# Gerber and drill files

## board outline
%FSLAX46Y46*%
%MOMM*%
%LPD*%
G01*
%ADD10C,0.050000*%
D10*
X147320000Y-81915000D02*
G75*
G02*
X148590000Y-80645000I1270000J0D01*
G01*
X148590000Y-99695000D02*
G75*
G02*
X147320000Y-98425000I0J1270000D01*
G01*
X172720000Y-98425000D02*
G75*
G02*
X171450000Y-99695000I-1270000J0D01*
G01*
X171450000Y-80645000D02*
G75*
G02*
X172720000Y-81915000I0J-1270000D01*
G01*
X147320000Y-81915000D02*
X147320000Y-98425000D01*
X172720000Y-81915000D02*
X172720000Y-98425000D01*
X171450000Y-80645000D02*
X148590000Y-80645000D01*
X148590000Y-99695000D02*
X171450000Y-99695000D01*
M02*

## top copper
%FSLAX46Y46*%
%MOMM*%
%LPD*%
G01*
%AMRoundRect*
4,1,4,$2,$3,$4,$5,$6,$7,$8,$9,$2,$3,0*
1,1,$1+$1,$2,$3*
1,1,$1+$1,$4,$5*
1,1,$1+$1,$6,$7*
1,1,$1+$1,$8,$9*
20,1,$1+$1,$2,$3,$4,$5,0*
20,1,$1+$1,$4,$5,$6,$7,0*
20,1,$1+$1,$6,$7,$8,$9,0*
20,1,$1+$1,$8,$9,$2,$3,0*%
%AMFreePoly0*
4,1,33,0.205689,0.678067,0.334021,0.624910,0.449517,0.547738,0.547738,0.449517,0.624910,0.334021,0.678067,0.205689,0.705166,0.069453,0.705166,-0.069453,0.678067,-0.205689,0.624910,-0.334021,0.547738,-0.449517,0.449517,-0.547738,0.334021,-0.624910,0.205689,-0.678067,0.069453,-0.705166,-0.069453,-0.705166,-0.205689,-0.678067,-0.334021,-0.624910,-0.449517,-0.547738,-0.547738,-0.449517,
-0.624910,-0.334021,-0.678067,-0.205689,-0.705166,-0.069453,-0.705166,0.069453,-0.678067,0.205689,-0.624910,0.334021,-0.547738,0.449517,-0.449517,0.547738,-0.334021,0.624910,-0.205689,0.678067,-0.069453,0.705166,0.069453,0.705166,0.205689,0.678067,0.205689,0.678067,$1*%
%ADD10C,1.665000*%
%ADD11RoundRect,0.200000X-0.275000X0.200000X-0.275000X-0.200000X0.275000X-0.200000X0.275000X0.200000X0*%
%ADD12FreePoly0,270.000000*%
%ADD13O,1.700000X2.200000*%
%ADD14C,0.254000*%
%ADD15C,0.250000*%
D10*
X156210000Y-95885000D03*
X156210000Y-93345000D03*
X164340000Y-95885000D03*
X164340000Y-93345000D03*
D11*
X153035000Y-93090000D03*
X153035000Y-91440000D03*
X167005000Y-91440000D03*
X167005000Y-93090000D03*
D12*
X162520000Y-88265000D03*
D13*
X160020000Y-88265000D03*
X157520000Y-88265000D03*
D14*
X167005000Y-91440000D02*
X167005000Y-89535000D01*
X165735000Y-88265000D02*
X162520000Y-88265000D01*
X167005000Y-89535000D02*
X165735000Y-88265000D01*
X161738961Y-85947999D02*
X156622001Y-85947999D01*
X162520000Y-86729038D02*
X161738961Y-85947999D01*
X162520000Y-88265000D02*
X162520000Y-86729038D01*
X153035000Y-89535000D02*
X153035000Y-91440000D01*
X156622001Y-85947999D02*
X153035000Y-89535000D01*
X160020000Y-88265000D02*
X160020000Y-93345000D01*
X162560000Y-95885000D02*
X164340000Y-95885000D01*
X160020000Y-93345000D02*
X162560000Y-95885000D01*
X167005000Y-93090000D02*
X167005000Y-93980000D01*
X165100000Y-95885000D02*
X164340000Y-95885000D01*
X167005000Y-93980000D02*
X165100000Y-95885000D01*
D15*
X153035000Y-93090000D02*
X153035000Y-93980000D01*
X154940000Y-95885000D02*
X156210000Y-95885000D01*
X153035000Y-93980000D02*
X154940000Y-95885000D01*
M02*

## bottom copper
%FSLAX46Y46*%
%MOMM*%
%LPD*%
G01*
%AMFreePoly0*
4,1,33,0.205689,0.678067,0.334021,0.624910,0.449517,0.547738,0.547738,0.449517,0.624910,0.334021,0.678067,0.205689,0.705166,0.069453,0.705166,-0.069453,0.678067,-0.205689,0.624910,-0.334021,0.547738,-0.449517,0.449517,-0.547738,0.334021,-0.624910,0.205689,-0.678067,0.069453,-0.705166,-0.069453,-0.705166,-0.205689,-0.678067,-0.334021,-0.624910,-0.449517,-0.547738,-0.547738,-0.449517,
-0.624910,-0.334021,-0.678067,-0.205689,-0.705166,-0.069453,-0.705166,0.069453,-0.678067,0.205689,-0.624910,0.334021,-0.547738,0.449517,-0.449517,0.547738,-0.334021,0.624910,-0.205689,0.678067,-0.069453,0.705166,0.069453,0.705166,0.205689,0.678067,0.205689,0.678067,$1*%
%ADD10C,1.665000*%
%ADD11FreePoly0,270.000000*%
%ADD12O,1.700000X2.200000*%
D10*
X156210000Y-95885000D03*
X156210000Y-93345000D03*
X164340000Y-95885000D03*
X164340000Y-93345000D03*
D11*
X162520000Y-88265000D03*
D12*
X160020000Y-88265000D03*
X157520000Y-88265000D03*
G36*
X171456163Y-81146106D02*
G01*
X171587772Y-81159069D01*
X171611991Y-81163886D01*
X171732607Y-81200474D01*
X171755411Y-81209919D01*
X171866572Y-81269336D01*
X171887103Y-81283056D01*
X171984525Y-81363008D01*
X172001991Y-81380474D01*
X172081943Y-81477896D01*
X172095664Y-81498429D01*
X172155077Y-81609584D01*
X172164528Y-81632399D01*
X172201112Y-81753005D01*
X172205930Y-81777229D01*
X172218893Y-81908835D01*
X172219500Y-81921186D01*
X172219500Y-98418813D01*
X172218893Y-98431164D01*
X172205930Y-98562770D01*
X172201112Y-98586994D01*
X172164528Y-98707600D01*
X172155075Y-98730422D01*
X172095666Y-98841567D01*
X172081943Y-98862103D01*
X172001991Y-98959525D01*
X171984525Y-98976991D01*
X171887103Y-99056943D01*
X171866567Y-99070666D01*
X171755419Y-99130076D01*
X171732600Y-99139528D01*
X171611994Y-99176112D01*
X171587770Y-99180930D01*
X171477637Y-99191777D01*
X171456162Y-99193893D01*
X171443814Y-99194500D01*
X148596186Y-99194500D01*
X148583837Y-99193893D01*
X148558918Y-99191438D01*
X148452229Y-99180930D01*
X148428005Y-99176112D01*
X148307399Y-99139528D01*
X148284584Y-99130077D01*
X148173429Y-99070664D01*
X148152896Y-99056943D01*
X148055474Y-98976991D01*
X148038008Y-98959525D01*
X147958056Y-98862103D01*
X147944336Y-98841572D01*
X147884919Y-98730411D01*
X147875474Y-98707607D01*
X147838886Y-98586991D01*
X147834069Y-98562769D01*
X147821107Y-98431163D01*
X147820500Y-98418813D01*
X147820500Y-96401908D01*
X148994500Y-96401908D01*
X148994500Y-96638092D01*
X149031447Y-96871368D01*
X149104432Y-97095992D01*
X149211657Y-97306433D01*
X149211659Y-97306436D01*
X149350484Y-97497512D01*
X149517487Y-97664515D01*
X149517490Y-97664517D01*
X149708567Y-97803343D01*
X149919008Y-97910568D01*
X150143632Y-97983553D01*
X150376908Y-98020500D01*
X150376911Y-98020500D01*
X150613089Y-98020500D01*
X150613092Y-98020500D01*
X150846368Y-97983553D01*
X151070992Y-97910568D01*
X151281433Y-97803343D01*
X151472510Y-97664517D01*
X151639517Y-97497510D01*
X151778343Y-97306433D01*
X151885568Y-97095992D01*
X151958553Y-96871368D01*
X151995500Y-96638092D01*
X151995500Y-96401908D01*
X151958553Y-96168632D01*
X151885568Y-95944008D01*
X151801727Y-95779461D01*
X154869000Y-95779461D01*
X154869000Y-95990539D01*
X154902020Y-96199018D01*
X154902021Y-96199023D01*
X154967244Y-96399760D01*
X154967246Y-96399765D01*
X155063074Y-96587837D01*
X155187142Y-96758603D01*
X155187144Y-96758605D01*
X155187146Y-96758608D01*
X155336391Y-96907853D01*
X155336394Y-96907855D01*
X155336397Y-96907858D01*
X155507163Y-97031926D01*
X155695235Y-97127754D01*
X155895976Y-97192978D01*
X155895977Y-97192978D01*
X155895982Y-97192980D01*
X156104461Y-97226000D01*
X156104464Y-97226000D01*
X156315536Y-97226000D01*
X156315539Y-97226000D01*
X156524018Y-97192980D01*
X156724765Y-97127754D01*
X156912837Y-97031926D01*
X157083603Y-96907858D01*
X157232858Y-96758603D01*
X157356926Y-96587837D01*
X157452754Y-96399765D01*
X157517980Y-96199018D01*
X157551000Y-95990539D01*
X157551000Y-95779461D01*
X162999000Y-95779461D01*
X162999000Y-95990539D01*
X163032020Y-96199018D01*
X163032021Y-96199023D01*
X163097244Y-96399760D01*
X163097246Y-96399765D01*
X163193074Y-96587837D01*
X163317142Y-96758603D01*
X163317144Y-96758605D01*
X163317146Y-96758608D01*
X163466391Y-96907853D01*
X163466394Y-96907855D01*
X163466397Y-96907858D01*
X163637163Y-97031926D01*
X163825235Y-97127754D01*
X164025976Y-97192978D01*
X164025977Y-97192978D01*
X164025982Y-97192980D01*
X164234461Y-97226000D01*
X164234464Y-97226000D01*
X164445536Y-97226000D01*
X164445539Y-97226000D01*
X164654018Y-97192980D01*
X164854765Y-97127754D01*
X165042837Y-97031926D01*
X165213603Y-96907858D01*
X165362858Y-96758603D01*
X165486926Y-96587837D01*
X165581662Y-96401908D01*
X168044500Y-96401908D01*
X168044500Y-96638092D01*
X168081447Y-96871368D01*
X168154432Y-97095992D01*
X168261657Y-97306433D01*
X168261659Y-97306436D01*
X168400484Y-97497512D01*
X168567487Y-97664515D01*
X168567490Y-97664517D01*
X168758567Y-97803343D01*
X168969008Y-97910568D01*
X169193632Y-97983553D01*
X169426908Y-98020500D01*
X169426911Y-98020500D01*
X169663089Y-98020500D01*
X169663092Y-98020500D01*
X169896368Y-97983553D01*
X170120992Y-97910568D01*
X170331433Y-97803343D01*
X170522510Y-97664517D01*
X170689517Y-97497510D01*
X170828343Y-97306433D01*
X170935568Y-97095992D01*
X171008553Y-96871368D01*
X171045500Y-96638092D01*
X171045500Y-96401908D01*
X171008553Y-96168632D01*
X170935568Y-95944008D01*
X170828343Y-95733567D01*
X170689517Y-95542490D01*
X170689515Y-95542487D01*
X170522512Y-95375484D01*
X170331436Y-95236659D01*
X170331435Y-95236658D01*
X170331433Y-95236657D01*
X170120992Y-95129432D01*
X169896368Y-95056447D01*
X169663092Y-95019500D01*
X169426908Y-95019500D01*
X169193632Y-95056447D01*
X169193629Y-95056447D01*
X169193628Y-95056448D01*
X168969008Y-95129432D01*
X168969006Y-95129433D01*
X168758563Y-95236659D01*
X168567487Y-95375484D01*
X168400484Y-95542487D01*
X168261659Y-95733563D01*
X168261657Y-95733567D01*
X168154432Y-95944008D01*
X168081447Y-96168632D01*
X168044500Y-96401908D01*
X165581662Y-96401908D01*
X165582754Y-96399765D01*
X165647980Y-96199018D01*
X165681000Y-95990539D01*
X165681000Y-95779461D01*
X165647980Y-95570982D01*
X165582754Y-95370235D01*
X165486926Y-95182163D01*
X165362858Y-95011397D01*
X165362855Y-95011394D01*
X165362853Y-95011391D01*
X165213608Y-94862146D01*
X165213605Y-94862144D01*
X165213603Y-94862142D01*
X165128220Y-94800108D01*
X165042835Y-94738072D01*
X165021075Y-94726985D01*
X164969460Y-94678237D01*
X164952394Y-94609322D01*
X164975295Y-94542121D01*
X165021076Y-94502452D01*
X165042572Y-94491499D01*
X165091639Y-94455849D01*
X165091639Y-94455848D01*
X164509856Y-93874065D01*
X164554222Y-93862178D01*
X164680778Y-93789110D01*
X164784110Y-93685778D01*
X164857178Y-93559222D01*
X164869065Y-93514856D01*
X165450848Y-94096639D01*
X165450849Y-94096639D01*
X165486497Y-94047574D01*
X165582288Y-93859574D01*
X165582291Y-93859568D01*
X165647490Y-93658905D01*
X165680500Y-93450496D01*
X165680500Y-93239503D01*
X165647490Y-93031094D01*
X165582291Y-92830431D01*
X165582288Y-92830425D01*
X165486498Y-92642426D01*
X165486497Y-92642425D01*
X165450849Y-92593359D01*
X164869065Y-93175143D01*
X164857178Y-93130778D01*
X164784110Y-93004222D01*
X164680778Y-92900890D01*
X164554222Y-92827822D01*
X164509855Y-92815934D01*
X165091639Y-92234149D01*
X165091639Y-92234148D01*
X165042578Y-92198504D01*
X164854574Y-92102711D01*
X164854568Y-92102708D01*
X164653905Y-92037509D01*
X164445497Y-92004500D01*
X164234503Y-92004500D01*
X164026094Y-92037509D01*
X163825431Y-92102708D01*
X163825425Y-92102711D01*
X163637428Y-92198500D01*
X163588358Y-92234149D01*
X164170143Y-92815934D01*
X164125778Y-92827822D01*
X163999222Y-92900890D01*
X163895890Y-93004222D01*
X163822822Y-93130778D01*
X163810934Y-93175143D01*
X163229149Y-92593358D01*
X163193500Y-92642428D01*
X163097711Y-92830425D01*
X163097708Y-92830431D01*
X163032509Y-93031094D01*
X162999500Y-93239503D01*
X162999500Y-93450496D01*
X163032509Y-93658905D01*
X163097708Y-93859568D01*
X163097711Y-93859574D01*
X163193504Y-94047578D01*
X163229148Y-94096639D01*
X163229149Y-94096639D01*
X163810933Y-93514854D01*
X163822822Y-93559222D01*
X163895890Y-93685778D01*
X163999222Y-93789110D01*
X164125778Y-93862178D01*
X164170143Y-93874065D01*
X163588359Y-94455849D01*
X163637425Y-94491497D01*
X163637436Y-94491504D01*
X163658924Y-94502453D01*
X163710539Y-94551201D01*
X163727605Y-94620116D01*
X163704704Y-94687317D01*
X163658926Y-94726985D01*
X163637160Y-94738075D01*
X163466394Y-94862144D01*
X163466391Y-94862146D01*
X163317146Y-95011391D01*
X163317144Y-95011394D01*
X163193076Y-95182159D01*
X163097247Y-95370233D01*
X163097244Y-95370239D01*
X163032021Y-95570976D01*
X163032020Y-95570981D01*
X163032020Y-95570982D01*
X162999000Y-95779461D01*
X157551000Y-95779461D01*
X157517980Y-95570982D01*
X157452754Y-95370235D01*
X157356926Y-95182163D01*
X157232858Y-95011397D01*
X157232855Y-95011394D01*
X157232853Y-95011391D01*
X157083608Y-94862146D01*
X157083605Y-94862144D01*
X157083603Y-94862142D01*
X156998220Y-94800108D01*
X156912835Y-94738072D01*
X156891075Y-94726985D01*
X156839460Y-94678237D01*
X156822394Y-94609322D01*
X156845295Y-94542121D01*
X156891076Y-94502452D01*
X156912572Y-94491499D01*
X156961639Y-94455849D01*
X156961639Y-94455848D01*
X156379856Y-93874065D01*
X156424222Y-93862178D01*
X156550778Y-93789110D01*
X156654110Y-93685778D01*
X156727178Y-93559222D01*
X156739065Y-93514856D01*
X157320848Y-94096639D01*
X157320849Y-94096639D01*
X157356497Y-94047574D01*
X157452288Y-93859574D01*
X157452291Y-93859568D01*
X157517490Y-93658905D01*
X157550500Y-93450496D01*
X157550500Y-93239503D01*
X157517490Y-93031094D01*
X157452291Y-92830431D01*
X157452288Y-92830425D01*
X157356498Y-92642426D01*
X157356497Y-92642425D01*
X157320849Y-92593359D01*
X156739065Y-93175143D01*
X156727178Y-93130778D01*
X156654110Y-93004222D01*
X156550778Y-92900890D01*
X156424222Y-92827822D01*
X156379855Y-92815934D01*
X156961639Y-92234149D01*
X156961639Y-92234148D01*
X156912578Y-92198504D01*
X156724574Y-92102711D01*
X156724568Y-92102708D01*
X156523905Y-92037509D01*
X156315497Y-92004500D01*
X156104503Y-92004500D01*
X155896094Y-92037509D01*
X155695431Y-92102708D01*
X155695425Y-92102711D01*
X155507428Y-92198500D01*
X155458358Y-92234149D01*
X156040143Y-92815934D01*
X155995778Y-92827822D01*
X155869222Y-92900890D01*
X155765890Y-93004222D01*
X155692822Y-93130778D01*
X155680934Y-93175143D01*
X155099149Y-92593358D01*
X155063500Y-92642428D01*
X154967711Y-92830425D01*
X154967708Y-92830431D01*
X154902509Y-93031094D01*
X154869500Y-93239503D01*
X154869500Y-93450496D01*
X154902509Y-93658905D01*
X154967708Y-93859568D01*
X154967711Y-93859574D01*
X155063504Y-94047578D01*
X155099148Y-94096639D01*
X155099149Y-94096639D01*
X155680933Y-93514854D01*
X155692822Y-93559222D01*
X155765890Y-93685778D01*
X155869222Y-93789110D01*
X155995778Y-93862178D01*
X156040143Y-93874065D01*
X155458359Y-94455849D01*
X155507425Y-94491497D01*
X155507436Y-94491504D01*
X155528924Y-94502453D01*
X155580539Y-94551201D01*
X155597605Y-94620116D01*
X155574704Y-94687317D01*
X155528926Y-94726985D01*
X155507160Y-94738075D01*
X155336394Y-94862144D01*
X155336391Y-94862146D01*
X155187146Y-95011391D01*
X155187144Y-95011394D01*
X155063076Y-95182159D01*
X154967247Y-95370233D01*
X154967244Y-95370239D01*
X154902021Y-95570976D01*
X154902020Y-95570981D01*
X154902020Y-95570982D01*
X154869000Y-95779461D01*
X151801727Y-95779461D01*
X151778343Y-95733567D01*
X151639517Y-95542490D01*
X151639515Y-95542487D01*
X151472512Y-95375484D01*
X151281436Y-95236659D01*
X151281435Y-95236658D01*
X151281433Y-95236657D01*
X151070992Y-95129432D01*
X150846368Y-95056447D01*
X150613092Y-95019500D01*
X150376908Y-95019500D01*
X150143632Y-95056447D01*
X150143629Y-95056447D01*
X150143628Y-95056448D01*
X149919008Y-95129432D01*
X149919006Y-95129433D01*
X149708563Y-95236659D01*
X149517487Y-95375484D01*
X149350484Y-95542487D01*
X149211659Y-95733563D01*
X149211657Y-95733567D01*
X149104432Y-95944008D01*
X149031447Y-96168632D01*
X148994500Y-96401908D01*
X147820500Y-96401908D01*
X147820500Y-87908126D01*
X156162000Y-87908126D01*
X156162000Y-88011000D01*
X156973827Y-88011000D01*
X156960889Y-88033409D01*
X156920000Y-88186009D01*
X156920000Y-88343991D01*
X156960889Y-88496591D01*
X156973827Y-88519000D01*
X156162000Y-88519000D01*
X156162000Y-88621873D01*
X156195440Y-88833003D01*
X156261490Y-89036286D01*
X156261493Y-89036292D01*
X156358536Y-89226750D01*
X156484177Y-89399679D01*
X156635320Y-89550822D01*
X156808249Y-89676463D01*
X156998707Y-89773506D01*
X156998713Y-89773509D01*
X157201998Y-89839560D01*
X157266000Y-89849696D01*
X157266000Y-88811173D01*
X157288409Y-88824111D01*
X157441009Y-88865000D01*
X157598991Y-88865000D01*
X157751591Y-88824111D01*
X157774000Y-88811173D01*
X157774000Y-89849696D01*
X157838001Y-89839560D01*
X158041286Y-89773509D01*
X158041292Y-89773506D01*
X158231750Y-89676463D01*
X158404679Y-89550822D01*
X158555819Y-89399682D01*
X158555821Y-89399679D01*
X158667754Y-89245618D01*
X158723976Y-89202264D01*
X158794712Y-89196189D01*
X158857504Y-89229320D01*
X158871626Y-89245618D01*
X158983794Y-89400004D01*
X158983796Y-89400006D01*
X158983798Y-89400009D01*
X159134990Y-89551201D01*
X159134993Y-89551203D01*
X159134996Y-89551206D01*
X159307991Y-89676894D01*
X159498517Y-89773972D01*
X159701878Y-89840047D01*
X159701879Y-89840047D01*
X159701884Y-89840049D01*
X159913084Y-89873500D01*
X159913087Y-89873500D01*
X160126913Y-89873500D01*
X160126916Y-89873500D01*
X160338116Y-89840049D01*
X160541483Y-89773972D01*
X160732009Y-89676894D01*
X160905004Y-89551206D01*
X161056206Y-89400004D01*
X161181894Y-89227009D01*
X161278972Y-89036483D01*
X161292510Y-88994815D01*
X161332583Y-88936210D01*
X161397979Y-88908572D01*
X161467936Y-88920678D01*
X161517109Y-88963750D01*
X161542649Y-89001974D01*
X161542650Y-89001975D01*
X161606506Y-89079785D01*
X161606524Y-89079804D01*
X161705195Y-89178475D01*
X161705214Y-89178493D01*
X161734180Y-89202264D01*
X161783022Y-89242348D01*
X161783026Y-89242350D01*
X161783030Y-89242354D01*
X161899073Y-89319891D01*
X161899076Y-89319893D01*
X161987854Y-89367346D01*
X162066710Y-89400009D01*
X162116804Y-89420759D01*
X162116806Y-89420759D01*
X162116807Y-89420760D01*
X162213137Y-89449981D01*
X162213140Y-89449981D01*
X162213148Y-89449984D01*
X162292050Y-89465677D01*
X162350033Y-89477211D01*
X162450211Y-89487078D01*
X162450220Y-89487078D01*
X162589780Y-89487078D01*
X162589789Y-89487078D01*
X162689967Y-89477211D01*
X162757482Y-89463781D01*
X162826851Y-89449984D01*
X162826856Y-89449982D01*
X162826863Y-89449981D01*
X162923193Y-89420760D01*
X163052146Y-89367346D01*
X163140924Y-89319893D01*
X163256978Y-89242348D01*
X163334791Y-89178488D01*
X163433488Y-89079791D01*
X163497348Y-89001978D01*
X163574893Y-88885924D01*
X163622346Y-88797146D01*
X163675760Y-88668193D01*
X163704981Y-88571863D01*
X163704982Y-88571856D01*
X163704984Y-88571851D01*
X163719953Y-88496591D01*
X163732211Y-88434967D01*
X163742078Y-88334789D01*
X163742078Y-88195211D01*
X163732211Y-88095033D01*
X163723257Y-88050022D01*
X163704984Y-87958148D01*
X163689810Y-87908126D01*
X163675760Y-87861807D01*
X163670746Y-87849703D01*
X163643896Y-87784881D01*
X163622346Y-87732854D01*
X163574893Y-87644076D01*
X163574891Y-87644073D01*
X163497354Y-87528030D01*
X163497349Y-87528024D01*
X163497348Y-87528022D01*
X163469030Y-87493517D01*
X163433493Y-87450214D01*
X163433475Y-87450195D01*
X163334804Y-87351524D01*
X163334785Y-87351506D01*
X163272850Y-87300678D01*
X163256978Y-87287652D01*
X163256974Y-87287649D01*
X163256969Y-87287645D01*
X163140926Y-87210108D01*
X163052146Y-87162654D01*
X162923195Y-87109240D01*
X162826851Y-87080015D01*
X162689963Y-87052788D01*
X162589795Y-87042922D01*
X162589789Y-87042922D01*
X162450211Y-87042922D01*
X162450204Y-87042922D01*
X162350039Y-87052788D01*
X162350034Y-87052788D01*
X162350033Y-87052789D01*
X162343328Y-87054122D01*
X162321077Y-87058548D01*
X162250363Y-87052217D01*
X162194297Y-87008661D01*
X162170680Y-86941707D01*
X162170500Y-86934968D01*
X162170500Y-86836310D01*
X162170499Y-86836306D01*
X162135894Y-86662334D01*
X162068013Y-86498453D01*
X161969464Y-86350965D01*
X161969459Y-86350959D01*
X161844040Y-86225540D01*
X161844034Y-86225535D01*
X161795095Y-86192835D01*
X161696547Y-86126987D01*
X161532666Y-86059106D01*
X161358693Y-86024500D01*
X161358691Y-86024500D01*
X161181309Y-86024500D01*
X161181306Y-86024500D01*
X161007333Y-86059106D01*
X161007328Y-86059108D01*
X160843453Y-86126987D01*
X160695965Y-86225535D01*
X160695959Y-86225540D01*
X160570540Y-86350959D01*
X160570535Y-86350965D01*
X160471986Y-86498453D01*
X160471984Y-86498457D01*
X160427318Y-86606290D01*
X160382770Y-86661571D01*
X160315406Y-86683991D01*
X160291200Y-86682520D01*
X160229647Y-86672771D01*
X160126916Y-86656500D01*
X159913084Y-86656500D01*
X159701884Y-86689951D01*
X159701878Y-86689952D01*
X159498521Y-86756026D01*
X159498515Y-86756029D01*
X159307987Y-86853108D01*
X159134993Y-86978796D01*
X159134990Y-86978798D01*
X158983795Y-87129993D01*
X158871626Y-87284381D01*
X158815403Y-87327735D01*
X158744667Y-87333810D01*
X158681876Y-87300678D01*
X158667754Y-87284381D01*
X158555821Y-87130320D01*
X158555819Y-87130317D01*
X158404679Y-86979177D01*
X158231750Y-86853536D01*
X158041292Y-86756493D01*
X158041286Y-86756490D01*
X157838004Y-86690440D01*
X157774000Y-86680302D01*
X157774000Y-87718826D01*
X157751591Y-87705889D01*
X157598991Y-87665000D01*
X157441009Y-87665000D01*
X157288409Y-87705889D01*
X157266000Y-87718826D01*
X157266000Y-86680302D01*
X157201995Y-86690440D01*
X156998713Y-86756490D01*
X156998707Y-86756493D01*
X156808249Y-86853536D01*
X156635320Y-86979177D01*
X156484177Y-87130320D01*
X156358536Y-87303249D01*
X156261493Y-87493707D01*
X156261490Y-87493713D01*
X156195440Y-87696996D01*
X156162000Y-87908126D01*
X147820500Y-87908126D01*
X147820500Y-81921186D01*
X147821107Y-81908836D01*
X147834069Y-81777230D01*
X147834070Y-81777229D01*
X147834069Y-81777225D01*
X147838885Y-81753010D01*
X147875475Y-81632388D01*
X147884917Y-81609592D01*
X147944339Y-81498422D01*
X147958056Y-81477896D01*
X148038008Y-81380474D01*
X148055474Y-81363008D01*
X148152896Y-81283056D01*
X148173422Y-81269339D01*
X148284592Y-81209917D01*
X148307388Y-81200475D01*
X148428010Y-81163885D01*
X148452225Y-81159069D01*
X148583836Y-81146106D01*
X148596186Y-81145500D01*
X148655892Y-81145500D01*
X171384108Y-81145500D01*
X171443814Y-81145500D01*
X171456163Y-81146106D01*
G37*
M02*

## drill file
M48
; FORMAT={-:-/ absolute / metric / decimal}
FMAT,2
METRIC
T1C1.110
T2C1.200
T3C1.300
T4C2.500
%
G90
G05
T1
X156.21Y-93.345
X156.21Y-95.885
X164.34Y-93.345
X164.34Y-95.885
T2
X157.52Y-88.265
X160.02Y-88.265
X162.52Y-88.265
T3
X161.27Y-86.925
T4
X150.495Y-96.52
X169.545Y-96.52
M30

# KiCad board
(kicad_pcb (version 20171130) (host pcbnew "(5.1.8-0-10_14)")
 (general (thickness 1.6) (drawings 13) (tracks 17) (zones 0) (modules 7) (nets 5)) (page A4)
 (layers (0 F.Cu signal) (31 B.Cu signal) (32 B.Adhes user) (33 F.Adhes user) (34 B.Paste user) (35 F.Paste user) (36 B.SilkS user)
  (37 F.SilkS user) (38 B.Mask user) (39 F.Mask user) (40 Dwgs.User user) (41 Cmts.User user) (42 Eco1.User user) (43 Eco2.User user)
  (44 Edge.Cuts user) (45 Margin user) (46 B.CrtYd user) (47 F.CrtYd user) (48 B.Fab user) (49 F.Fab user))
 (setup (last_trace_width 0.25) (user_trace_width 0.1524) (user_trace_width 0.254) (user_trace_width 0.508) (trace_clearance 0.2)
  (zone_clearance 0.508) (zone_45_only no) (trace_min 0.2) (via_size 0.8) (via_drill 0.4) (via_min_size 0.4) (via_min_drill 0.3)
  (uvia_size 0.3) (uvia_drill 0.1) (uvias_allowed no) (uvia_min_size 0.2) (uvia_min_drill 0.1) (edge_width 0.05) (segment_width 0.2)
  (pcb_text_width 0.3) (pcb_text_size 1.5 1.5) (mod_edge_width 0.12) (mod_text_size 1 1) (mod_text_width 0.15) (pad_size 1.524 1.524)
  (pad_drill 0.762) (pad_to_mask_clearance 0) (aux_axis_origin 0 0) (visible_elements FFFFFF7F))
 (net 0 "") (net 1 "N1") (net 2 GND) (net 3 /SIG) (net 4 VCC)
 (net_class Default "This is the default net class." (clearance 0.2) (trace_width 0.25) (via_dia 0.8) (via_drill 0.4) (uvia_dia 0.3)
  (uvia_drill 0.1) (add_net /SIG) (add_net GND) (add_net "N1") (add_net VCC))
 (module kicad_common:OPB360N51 (layer B.Cu) (at 156.21 93.345)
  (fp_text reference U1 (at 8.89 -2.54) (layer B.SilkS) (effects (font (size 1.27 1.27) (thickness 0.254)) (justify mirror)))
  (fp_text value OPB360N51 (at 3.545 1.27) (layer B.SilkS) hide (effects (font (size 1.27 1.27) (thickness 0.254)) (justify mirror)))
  (pad 1 thru_hole circle (at 0 2.54) (size 1.665 1.665) (drill 1.11) (layers *.Cu *.Mask) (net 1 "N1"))
  (pad 2 thru_hole circle (at 0 0) (size 1.665 1.665) (drill 1.11) (layers *.Cu *.Mask) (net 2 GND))
  (pad 3 thru_hole circle (at 8.13 2.54) (size 1.665 1.665) (drill 1.11) (layers *.Cu *.Mask) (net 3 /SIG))
  (pad 4 thru_hole circle (at 8.13 0) (size 1.665 1.665) (drill 1.11) (layers *.Cu *.Mask) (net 2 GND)))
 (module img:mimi (layer F.Cu) (at 169.672 84.836)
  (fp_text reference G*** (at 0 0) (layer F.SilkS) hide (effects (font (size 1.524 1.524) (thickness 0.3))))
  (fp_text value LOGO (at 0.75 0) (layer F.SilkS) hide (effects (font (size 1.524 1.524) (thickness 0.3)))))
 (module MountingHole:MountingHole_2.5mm (layer F.Cu) (at 169.545 96.52)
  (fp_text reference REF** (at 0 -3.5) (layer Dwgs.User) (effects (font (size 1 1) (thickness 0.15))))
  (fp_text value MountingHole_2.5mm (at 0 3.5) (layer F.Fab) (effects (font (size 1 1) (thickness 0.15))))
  (pad 1 np_thru_hole circle (at 0 0) (size 2.5 2.5) (drill 2.5) (layers *.Cu *.Mask)))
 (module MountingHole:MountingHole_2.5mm (layer F.Cu) (at 150.495 96.52)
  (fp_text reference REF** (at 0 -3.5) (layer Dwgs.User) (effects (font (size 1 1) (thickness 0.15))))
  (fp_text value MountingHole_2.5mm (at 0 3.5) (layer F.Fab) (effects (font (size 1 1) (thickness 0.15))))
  (pad 1 np_thru_hole circle (at 0 0) (size 2.5 2.5) (drill 2.5) (layers *.Cu *.Mask)))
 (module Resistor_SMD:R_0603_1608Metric (layer F.Cu) (at 153.035 92.265 270)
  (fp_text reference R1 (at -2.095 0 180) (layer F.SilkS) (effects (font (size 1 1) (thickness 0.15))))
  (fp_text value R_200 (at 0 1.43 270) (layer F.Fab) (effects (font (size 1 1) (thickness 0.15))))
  (pad 2 smd roundrect (at 0.825 0 270) (size 0.8 0.95) (layers F.Cu F.Paste F.Mask) (roundrect_rratio 0.25) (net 1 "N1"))
  (pad 1 smd roundrect (at -0.825 0 270) (size 0.8 0.95) (layers F.Cu F.Paste F.Mask) (roundrect_rratio 0.25) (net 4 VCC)))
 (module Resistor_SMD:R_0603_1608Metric (layer F.Cu) (at 167.005 92.265 270)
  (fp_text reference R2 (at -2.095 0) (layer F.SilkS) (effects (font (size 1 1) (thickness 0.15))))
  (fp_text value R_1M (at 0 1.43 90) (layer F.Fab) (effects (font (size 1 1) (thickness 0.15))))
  (pad 1 smd roundrect (at -0.825 0 270) (size 0.8 0.95) (layers F.Cu F.Paste F.Mask) (roundrect_rratio 0.25) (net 4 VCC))
  (pad 2 smd roundrect (at 0.825 0 270) (size 0.8 0.95) (layers F.Cu F.Paste F.Mask) (roundrect_rratio 0.25) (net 3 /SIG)))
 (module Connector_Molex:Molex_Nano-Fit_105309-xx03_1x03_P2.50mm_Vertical (layer F.Cu) (at 162.52 88.265 270)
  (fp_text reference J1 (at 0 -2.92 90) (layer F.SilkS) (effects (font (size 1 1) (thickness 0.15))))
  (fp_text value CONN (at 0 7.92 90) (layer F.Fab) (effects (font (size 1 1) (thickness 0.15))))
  (pad 1 thru_hole custom (at 0 0 270) (size 1.417157 1.417157) (drill 1.2) (layers *.Cu *.Mask) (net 4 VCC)
   (options (clearance outline) (anchor circle)) (primitives))
  (pad 2 thru_hole oval (at 0 2.5 270) (size 2.2 1.7) (drill 1.2) (layers *.Cu *.Mask) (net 3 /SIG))
  (pad 3 thru_hole oval (at 0 5 270) (size 2.2 1.7) (drill 1.2) (layers *.Cu *.Mask) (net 2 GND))
  (pad "" np_thru_hole circle (at -1.34 1.25 270) (size 1.3 1.3) (drill 1.3) (layers *.Cu *.Mask)))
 (gr_arc (start 148.59 81.915) (end 148.59 80.645) (angle -90) (layer Edge.Cuts) (width 0.05))
 (gr_arc (start 148.59 98.425) (end 147.32 98.425) (angle -90) (layer Edge.Cuts) (width 0.05))
 (gr_arc (start 171.45 98.425) (end 171.45 99.695) (angle -90) (layer Edge.Cuts) (width 0.05))
 (gr_arc (start 171.45 81.915) (end 172.72 81.915) (angle -90) (layer Edge.Cuts) (width 0.05))
 (gr_line (start 147.32 81.915) (end 147.32 98.425) (layer Edge.Cuts) (width 0.05))
 (gr_line (start 172.72 81.915) (end 172.72 98.425) (layer Edge.Cuts) (width 0.05))
 (gr_line (start 171.45 80.645) (end 148.59 80.645) (layer Edge.Cuts) (width 0.05))
 (gr_line (start 148.59 99.695) (end 171.45 99.695) (layer Edge.Cuts) (width 0.05))
 (segment (start 167.005 91.44) (end 167.005 89.535) (width 0.254) (layer F.Cu) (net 4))
 (segment (start 165.735 88.265) (end 162.52 88.265) (width 0.254) (layer F.Cu) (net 4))
 (segment (start 167.005 89.535) (end 165.735 88.265) (width 0.254) (layer F.Cu) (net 4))
 (segment (start 161.738961 85.947999) (end 156.622001 85.947999) (width 0.254) (layer F.Cu) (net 4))
 (segment (start 162.52 86.729038) (end 161.738961 85.947999) (width 0.254) (layer F.Cu) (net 4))
 (segment (start 162.52 88.265) (end 162.52 86.729038) (width 0.254) (layer F.Cu) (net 4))
 (segment (start 153.035 89.535) (end 153.035 91.44) (width 0.254) (layer F.Cu) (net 4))
 (segment (start 156.622001 85.947999) (end 153.035 89.535) (width 0.254) (layer F.Cu) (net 4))
 (segment (start 160.02 88.265) (end 160.02 93.345) (width 0.254) (layer F.Cu) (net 3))
 (segment (start 162.56 95.885) (end 164.34 95.885) (width 0.254) (layer F.Cu) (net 3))
 (segment (start 160.02 93.345) (end 162.56 95.885) (width 0.254) (layer F.Cu) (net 3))
 (segment (start 167.005 93.09) (end 167.005 93.98) (width 0.254) (layer F.Cu) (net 3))
 (segment (start 165.1 95.885) (end 164.34 95.885) (width 0.254) (layer F.Cu) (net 3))
 (segment (start 167.005 93.98) (end 165.1 95.885) (width 0.254) (layer F.Cu) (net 3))
 (segment (start 153.035 93.09) (end 153.035 93.98) (width 0.25) (layer F.Cu) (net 1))
 (segment (start 154.94 95.885) (end 156.21 95.885) (width 0.25) (layer F.Cu) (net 1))
 (segment (start 153.035 93.98) (end 154.94 95.885) (width 0.25) (layer F.Cu) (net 1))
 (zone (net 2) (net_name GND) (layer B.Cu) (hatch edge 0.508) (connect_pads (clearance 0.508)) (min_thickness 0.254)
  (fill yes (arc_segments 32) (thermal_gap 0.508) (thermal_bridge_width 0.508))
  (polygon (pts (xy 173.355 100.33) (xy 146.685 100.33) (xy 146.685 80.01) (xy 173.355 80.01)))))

